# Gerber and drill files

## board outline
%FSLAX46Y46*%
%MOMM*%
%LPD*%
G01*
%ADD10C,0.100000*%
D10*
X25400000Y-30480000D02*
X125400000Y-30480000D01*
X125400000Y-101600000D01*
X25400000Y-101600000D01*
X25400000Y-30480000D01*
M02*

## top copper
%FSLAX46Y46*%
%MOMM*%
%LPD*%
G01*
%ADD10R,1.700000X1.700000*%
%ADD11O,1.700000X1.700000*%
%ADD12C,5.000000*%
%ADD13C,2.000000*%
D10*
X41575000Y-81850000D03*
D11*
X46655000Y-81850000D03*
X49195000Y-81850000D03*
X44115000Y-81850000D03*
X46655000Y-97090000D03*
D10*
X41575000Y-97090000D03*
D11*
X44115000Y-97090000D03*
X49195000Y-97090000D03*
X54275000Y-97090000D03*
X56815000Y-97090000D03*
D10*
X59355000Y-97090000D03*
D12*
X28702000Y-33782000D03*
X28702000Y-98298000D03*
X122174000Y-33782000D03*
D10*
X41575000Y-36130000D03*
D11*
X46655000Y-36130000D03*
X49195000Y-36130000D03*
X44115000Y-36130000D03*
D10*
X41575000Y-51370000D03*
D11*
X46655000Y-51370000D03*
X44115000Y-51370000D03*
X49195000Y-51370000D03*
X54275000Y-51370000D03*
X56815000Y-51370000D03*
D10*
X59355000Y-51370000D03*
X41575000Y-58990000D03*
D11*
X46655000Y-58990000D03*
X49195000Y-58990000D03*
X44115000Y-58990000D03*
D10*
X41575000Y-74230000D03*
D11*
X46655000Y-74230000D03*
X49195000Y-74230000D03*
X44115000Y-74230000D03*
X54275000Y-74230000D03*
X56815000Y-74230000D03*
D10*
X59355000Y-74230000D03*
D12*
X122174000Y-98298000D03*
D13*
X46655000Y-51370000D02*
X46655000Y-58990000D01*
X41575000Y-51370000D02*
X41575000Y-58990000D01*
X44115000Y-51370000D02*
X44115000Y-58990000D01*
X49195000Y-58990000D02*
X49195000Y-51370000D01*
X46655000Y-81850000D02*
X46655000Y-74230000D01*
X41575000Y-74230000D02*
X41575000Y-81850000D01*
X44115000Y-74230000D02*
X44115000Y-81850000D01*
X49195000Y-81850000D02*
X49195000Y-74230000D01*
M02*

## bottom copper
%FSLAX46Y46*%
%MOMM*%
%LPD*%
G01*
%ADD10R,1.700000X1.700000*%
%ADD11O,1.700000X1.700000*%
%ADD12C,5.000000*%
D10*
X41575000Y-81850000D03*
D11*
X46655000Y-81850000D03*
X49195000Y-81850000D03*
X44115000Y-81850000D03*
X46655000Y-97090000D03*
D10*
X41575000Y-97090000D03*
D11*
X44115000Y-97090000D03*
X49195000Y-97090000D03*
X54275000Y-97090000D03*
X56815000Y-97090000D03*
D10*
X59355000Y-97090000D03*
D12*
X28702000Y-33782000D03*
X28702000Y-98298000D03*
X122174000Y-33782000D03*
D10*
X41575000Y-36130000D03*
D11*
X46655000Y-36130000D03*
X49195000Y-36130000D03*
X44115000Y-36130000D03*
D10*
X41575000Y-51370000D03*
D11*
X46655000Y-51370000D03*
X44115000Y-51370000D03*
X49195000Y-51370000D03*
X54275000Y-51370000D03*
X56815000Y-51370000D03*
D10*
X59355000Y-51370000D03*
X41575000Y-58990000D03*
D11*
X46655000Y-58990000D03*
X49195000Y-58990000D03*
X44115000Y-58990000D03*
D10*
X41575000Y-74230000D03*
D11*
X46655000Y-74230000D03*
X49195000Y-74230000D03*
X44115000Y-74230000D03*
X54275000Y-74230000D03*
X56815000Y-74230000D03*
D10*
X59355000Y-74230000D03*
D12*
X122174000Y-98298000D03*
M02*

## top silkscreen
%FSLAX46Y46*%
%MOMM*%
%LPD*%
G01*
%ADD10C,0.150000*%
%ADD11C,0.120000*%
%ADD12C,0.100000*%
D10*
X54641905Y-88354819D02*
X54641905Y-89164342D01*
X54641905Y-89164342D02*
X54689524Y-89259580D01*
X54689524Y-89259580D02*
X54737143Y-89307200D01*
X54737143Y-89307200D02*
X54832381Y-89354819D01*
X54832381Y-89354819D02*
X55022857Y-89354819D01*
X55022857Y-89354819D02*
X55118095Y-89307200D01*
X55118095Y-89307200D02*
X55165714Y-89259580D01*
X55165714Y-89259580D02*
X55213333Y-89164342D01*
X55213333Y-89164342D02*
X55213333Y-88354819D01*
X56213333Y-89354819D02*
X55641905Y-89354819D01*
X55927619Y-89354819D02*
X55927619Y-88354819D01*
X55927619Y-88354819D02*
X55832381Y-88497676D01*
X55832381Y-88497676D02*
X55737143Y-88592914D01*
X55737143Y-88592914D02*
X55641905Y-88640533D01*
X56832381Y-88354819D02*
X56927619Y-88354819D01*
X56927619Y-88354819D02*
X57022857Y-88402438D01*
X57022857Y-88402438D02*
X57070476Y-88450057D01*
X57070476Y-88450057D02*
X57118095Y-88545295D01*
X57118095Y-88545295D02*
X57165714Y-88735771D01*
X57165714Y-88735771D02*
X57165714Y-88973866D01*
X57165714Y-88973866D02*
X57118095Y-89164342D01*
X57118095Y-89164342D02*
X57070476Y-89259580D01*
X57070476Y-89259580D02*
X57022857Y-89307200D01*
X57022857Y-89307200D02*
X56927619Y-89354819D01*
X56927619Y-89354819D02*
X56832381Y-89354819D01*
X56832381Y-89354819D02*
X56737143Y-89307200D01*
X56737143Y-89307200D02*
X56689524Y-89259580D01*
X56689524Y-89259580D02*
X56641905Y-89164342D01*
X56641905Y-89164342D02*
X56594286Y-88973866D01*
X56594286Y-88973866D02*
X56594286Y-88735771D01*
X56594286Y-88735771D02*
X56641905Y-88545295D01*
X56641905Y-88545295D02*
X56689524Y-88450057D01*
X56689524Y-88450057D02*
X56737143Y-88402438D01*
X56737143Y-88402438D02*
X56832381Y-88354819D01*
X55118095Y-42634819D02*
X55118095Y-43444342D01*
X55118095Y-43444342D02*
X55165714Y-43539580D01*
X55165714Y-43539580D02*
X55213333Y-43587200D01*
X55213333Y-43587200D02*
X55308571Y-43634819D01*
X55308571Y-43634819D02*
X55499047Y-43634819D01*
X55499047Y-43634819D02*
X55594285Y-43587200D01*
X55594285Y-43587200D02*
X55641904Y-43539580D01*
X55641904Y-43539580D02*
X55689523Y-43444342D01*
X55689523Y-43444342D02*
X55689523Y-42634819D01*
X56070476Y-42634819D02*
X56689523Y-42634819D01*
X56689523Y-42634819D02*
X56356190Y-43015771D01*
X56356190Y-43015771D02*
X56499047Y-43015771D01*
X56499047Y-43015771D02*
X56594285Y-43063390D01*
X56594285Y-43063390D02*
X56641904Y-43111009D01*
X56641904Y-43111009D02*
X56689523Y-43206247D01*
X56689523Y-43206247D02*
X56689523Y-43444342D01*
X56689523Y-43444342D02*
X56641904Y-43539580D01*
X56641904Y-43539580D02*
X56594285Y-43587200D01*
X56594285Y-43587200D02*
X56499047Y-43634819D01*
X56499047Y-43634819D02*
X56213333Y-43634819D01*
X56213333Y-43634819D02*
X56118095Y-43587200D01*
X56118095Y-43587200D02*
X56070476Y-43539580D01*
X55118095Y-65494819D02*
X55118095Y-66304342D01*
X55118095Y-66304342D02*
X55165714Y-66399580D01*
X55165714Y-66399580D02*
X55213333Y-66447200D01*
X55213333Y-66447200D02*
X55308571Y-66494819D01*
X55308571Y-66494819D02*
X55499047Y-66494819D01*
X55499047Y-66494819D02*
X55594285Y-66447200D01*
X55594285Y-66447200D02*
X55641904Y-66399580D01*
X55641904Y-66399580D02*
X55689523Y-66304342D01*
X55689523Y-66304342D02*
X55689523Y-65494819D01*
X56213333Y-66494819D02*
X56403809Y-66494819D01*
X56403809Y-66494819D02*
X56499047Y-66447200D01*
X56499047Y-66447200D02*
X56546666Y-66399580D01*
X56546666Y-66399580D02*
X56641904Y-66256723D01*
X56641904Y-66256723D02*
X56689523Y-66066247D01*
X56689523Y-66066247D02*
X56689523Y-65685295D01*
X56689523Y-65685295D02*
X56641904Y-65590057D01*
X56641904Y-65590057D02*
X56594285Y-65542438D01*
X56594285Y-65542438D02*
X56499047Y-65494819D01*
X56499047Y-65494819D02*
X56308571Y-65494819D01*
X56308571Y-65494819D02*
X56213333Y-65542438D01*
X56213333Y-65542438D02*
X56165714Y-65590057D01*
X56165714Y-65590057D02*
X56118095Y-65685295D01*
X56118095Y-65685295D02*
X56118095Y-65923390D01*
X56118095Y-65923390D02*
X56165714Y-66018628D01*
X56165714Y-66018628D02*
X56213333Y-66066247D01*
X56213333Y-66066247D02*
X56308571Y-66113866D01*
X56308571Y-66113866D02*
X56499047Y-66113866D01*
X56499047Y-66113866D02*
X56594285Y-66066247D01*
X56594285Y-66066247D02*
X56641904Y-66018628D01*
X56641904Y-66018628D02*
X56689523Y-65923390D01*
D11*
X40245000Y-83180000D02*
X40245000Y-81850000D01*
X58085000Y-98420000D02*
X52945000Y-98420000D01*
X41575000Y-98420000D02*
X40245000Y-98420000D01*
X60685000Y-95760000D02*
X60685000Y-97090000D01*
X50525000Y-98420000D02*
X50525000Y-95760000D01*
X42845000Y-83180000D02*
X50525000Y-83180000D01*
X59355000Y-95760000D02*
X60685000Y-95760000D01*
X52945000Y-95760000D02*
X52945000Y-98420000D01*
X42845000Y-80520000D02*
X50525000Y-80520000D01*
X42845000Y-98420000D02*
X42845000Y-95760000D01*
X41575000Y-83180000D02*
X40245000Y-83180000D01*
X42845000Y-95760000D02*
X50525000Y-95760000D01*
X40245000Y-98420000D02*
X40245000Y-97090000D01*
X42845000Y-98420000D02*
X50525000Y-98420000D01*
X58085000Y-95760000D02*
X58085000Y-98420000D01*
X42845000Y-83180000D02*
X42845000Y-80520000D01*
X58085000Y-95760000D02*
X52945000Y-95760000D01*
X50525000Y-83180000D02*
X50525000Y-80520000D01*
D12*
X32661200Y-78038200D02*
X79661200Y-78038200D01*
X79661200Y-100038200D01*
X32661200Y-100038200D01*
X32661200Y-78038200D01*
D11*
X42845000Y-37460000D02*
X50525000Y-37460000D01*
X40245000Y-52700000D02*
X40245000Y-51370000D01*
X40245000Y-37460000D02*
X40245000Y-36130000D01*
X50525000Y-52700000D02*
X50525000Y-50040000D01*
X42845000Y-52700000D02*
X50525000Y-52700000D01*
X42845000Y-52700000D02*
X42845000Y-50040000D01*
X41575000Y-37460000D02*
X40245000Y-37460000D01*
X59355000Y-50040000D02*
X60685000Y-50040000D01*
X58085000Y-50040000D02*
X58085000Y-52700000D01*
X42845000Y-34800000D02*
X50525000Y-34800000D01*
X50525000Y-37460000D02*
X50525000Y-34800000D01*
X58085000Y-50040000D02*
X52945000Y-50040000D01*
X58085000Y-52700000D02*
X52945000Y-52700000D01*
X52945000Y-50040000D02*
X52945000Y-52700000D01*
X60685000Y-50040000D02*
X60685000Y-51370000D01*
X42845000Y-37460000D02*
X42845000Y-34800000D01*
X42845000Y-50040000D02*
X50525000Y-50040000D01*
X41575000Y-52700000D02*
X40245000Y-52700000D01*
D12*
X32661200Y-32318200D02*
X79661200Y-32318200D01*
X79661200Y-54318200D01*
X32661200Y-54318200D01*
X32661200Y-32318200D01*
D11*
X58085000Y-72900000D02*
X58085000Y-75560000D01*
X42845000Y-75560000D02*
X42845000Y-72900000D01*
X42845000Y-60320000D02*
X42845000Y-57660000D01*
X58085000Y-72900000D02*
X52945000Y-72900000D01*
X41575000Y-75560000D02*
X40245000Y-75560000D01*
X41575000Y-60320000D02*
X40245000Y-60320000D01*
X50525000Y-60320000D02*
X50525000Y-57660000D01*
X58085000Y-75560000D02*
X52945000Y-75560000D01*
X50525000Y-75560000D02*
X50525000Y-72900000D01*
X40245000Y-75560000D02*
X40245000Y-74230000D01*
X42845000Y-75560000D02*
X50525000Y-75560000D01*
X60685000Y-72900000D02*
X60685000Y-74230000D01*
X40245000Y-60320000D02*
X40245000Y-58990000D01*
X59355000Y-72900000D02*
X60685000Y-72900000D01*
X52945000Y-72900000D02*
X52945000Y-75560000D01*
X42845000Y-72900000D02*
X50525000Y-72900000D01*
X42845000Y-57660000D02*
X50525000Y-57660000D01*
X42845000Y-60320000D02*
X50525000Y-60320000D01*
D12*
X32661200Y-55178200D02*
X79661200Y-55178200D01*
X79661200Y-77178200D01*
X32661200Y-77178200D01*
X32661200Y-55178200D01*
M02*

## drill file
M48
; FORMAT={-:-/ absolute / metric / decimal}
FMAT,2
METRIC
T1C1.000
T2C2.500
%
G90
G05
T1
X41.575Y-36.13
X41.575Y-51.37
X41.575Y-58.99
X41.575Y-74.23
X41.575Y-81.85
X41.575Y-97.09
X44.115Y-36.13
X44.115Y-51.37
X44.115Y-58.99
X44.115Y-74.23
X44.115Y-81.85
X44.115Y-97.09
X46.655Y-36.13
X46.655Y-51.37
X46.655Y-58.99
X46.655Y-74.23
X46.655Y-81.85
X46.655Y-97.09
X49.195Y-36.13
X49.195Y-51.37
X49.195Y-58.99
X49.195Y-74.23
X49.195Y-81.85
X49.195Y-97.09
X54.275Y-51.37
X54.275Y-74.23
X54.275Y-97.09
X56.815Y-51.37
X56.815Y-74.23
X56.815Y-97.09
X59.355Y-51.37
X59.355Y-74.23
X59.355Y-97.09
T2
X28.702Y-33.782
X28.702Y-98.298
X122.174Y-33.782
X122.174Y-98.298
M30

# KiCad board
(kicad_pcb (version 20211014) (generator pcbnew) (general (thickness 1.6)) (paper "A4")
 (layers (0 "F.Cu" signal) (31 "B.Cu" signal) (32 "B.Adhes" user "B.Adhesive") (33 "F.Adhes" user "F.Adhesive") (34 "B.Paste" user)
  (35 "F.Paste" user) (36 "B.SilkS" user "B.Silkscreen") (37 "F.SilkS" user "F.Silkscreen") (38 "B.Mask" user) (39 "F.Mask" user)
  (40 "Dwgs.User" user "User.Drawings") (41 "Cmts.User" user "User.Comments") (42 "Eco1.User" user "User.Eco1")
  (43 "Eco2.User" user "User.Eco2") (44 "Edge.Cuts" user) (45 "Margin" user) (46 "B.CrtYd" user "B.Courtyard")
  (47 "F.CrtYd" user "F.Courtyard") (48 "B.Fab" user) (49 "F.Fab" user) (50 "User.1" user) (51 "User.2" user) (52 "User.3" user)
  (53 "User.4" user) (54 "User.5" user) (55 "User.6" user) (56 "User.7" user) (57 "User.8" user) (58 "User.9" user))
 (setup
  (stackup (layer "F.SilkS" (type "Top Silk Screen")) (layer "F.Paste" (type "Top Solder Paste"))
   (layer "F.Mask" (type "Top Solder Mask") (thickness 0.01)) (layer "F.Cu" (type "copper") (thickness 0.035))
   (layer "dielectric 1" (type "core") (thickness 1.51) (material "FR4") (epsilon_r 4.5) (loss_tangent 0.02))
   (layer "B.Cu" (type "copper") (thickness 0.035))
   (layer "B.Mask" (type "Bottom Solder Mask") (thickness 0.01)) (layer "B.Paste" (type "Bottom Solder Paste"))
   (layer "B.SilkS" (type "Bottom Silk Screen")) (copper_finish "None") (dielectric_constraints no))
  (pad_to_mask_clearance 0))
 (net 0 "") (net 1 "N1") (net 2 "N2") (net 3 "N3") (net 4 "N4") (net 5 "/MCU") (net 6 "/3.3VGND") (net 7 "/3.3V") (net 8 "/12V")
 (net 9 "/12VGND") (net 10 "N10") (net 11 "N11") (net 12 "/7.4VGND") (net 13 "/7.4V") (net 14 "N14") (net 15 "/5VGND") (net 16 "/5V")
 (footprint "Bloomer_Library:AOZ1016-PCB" (layer "F.Cu") (at 55.88 88.9)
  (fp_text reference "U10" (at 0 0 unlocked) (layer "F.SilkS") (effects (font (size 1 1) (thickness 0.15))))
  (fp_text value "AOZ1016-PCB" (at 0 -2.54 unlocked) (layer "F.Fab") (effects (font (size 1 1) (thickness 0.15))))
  (fp_line (start -15.635 -5.72) (end -15.635 -7.05) (layer "F.SilkS") (width 0.12))
  (fp_line (start 2.205 9.52) (end -2.935 9.52) (layer "F.SilkS") (width 0.12))
  (fp_line (start -14.305 9.52) (end -15.635 9.52) (layer "F.SilkS") (width 0.12))
  (fp_line (start 4.805 6.86) (end 4.805 8.19) (layer "F.SilkS") (width 0.12))
  (fp_line (start -5.355 9.52) (end -5.355 6.86) (layer "F.SilkS") (width 0.12))
  (fp_line (start -13.035 -5.72) (end -5.355 -5.72) (layer "F.SilkS") (width 0.12))
  (fp_line (start 3.475 6.86) (end 4.805 6.86) (layer "F.SilkS") (width 0.12))
  (fp_line (start -2.935 6.86) (end -2.935 9.52) (layer "F.SilkS") (width 0.12))
  (fp_line (start -13.035 -8.38) (end -5.355 -8.38) (layer "F.SilkS") (width 0.12))
  (fp_line (start -13.035 9.52) (end -13.035 6.86) (layer "F.SilkS") (width 0.12))
  (fp_line (start -14.305 -5.72) (end -15.635 -5.72) (layer "F.SilkS") (width 0.12))
  (fp_line (start -13.035 6.86) (end -5.355 6.86) (layer "F.SilkS") (width 0.12))
  (fp_line (start -15.635 9.52) (end -15.635 8.19) (layer "F.SilkS") (width 0.12))
  (fp_line (start -13.035 9.52) (end -5.355 9.52) (layer "F.SilkS") (width 0.12))
  (fp_line (start 2.205 6.86) (end 2.205 9.52) (layer "F.SilkS") (width 0.12))
  (fp_line (start -13.035 -5.72) (end -13.035 -8.38) (layer "F.SilkS") (width 0.12))
  (fp_line (start 2.205 6.86) (end -2.935 6.86) (layer "F.SilkS") (width 0.12))
  (fp_line (start -5.355 -5.72) (end -5.355 -8.38) (layer "F.SilkS") (width 0.12))
  (fp_rect (start 23.7812 -10.8618) (end -23.2188 11.1382) (layer "F.SilkS") (width 0.1) (fill none))
  (pad "3" thru_hole rect (at -14.305 -7.05 90) (size 1.7 1.7) (drill 1) (layers *.Cu *.Mask) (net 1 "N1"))
  (pad "3" thru_hole oval (at -9.225 -7.05 90) (size 1.7 1.7) (drill 1) (layers *.Cu *.Mask) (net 1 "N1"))
  (pad "4" thru_hole oval (at -6.685 -7.05 90) (size 1.7 1.7) (drill 1) (layers *.Cu *.Mask) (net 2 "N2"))
  (pad "4" thru_hole oval (at -11.765 -7.05 90) (size 1.7 1.7) (drill 1) (layers *.Cu *.Mask) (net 2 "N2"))
  (pad "5" thru_hole oval (at -9.225 8.19 90) (size 1.7 1.7) (drill 1) (layers *.Cu *.Mask) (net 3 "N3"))
  (pad "5" thru_hole rect (at -14.305 8.19 90) (size 1.7 1.7) (drill 1) (layers *.Cu *.Mask) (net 3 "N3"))
  (pad "6" thru_hole oval (at -11.765 8.19 90) (size 1.7 1.7) (drill 1) (layers *.Cu *.Mask) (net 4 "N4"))
  (pad "6" thru_hole oval (at -6.685 8.19 90) (size 1.7 1.7) (drill 1) (layers *.Cu *.Mask) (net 4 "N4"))
  (pad "7" thru_hole oval (at -1.605 8.19 270) (size 1.7 1.7) (drill 1) (layers *.Cu *.Mask) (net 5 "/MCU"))
  (pad "8" thru_hole oval (at 0.935 8.19 270) (size 1.7 1.7) (drill 1) (layers *.Cu *.Mask) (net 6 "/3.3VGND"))
  (pad "9" thru_hole rect (at 3.475 8.19 270) (size 1.7 1.7) (drill 1) (layers *.Cu *.Mask) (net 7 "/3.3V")))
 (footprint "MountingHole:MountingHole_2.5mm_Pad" (layer "F.Cu") (at 28.702 33.782)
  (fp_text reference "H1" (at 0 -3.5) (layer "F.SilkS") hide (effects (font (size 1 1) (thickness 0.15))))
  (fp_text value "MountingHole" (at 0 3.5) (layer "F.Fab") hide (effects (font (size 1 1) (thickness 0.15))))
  (pad "1" thru_hole circle (at 0 0) (size 5 5) (drill 2.5) (layers *.Cu *.Mask)))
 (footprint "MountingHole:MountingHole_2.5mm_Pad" (layer "F.Cu") (at 28.702 98.298)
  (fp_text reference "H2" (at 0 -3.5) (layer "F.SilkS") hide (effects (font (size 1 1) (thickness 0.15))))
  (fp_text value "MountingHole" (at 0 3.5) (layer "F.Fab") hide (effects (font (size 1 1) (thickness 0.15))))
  (pad "1" thru_hole circle (at 0 0) (size 5 5) (drill 2.5) (layers *.Cu *.Mask)))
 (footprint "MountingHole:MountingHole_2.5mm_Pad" (layer "F.Cu") (at 122.174 33.782)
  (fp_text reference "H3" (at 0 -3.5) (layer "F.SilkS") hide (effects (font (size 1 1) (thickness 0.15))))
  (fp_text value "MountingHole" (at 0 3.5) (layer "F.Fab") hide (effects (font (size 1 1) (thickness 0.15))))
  (pad "1" thru_hole circle (at 0 0) (size 5 5) (drill 2.5) (layers *.Cu *.Mask)))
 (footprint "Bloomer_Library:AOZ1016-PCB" (layer "F.Cu") (at 55.88 43.18)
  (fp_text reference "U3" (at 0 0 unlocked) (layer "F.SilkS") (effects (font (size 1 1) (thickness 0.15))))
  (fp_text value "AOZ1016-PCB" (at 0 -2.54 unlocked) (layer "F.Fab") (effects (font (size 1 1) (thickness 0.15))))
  (fp_line (start -13.035 -5.72) (end -5.355 -5.72) (layer "F.SilkS") (width 0.12))
  (fp_line (start -15.635 9.52) (end -15.635 8.19) (layer "F.SilkS") (width 0.12))
  (fp_line (start -15.635 -5.72) (end -15.635 -7.05) (layer "F.SilkS") (width 0.12))
  (fp_line (start -5.355 9.52) (end -5.355 6.86) (layer "F.SilkS") (width 0.12))
  (fp_line (start -13.035 9.52) (end -5.355 9.52) (layer "F.SilkS") (width 0.12))
  (fp_line (start -13.035 9.52) (end -13.035 6.86) (layer "F.SilkS") (width 0.12))
  (fp_line (start -14.305 -5.72) (end -15.635 -5.72) (layer "F.SilkS") (width 0.12))
  (fp_line (start 3.475 6.86) (end 4.805 6.86) (layer "F.SilkS") (width 0.12))
  (fp_line (start 2.205 6.86) (end 2.205 9.52) (layer "F.SilkS") (width 0.12))
  (fp_line (start -13.035 -8.38) (end -5.355 -8.38) (layer "F.SilkS") (width 0.12))
  (fp_line (start -5.355 -5.72) (end -5.355 -8.38) (layer "F.SilkS") (width 0.12))
  (fp_line (start 2.205 6.86) (end -2.935 6.86) (layer "F.SilkS") (width 0.12))
  (fp_line (start 2.205 9.52) (end -2.935 9.52) (layer "F.SilkS") (width 0.12))
  (fp_line (start -2.935 6.86) (end -2.935 9.52) (layer "F.SilkS") (width 0.12))
  (fp_line (start 4.805 6.86) (end 4.805 8.19) (layer "F.SilkS") (width 0.12))
  (fp_line (start -13.035 -5.72) (end -13.035 -8.38) (layer "F.SilkS") (width 0.12))
  (fp_line (start -13.035 6.86) (end -5.355 6.86) (layer "F.SilkS") (width 0.12))
  (fp_line (start -14.305 9.52) (end -15.635 9.52) (layer "F.SilkS") (width 0.12))
  (fp_rect (start 23.7812 -10.8618) (end -23.2188 11.1382) (layer "F.SilkS") (width 0.1) (fill none))
  (pad "3" thru_hole rect (at -14.305 -7.05 90) (size 1.7 1.7) (drill 1) (layers *.Cu *.Mask) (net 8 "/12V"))
  (pad "3" thru_hole oval (at -9.225 -7.05 90) (size 1.7 1.7) (drill 1) (layers *.Cu *.Mask) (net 8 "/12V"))
  (pad "4" thru_hole oval (at -6.685 -7.05 90) (size 1.7 1.7) (drill 1) (layers *.Cu *.Mask) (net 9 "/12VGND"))
  (pad "4" thru_hole oval (at -11.765 -7.05 90) (size 1.7 1.7) (drill 1) (layers *.Cu *.Mask) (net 9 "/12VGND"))
  (pad "5" thru_hole rect (at -14.305 8.19 90) (size 1.7 1.7) (drill 1) (layers *.Cu *.Mask) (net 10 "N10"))
  (pad "5" thru_hole oval (at -9.225 8.19 90) (size 1.7 1.7) (drill 1) (layers *.Cu *.Mask) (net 10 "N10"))
  (pad "6" thru_hole oval (at -11.765 8.19 90) (size 1.7 1.7) (drill 1) (layers *.Cu *.Mask) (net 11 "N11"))
  (pad "6" thru_hole oval (at -6.685 8.19 90) (size 1.7 1.7) (drill 1) (layers *.Cu *.Mask) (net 11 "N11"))
  (pad "7" thru_hole oval (at -1.605 8.19 270) (size 1.7 1.7) (drill 1) (layers *.Cu *.Mask) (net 5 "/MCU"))
  (pad "8" thru_hole oval (at 0.935 8.19 270) (size 1.7 1.7) (drill 1) (layers *.Cu *.Mask) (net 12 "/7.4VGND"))
  (pad "9" thru_hole rect (at 3.475 8.19 270) (size 1.7 1.7) (drill 1) (layers *.Cu *.Mask) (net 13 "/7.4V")))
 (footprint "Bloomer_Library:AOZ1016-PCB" (layer "F.Cu") (at 55.88 66.04)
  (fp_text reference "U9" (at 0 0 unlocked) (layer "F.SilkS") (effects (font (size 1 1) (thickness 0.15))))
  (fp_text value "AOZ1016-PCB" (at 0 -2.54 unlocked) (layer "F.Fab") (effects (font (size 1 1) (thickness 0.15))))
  (fp_line (start 2.205 6.86) (end 2.205 9.52) (layer "F.SilkS") (width 0.12))
  (fp_line (start -13.035 9.52) (end -13.035 6.86) (layer "F.SilkS") (width 0.12))
  (fp_line (start -13.035 -5.72) (end -13.035 -8.38) (layer "F.SilkS") (width 0.12))
  (fp_line (start 2.205 6.86) (end -2.935 6.86) (layer "F.SilkS") (width 0.12))
  (fp_line (start -14.305 9.52) (end -15.635 9.52) (layer "F.SilkS") (width 0.12))
  (fp_line (start -14.305 -5.72) (end -15.635 -5.72) (layer "F.SilkS") (width 0.12))
  (fp_line (start -5.355 -5.72) (end -5.355 -8.38) (layer "F.SilkS") (width 0.12))
  (fp_line (start 2.205 9.52) (end -2.935 9.52) (layer "F.SilkS") (width 0.12))
  (fp_line (start -5.355 9.52) (end -5.355 6.86) (layer "F.SilkS") (width 0.12))
  (fp_line (start -15.635 9.52) (end -15.635 8.19) (layer "F.SilkS") (width 0.12))
  (fp_line (start -13.035 9.52) (end -5.355 9.52) (layer "F.SilkS") (width 0.12))
  (fp_line (start 4.805 6.86) (end 4.805 8.19) (layer "F.SilkS") (width 0.12))
  (fp_line (start -15.635 -5.72) (end -15.635 -7.05) (layer "F.SilkS") (width 0.12))
  (fp_line (start 3.475 6.86) (end 4.805 6.86) (layer "F.SilkS") (width 0.12))
  (fp_line (start -2.935 6.86) (end -2.935 9.52) (layer "F.SilkS") (width 0.12))
  (fp_line (start -13.035 6.86) (end -5.355 6.86) (layer "F.SilkS") (width 0.12))
  (fp_line (start -13.035 -8.38) (end -5.355 -8.38) (layer "F.SilkS") (width 0.12))
  (fp_line (start -13.035 -5.72) (end -5.355 -5.72) (layer "F.SilkS") (width 0.12))
  (fp_rect (start 23.7812 -10.8618) (end -23.2188 11.1382) (layer "F.SilkS") (width 0.1) (fill none))
  (pad "3" thru_hole rect (at -14.305 -7.05 90) (size 1.7 1.7) (drill 1) (layers *.Cu *.Mask) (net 10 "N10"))
  (pad "3" thru_hole oval (at -9.225 -7.05 90) (size 1.7 1.7) (drill 1) (layers *.Cu *.Mask) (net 10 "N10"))
  (pad "4" thru_hole oval (at -6.685 -7.05 90) (size 1.7 1.7) (drill 1) (layers *.Cu *.Mask) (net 11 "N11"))
  (pad "4" thru_hole oval (at -11.765 -7.05 90) (size 1.7 1.7) (drill 1) (layers *.Cu *.Mask) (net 11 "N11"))
  (pad "5" thru_hole rect (at -14.305 8.19 90) (size 1.7 1.7) (drill 1) (layers *.Cu *.Mask) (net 1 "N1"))
  (pad "5" thru_hole oval (at -9.225 8.19 90) (size 1.7 1.7) (drill 1) (layers *.Cu *.Mask) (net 1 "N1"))
  (pad "6" thru_hole oval (at -6.685 8.19 90) (size 1.7 1.7) (drill 1) (layers *.Cu *.Mask) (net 2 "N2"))
  (pad "6" thru_hole oval (at -11.765 8.19 90) (size 1.7 1.7) (drill 1) (layers *.Cu *.Mask) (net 2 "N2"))
  (pad "7" thru_hole oval (at -1.605 8.19 270) (size 1.7 1.7) (drill 1) (layers *.Cu *.Mask) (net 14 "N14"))
  (pad "8" thru_hole oval (at 0.935 8.19 270) (size 1.7 1.7) (drill 1) (layers *.Cu *.Mask) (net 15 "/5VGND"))
  (pad "9" thru_hole rect (at 3.475 8.19 270) (size 1.7 1.7) (drill 1) (layers *.Cu *.Mask) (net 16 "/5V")))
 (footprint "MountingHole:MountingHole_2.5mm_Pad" (layer "F.Cu") (at 122.174 98.298)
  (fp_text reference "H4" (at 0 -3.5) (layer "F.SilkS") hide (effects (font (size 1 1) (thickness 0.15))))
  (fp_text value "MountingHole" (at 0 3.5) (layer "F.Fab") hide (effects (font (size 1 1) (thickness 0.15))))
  (pad "1" thru_hole circle (at 0 0) (size 5 5) (drill 2.5) (layers *.Cu *.Mask)))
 (gr_rect (start 25.4 30.48) (end 125.4 101.6) (layer "Edge.Cuts") (width 0.1) (fill none))
 (segment (start 46.655 51.37) (end 46.655 58.99) (width 2) (layer "F.Cu") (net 10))
 (segment (start 41.575 51.37) (end 41.575 58.99) (width 2) (layer "F.Cu") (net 10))
 (segment (start 44.115 51.37) (end 44.115 58.99) (width 2) (layer "F.Cu") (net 11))
 (segment (start 49.195 58.99) (end 49.195 51.37) (width 2) (layer "F.Cu") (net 11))
 (segment (start 46.655 81.85) (end 46.655 74.23) (width 2) (layer "F.Cu") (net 1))
 (segment (start 41.575 74.23) (end 41.575 81.85) (width 2) (layer "F.Cu") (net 1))
 (segment (start 44.115 74.23) (end 44.115 81.85) (width 2) (layer "F.Cu") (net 2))
 (segment (start 49.195 81.85) (end 49.195 74.23) (width 2) (layer "F.Cu") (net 2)))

